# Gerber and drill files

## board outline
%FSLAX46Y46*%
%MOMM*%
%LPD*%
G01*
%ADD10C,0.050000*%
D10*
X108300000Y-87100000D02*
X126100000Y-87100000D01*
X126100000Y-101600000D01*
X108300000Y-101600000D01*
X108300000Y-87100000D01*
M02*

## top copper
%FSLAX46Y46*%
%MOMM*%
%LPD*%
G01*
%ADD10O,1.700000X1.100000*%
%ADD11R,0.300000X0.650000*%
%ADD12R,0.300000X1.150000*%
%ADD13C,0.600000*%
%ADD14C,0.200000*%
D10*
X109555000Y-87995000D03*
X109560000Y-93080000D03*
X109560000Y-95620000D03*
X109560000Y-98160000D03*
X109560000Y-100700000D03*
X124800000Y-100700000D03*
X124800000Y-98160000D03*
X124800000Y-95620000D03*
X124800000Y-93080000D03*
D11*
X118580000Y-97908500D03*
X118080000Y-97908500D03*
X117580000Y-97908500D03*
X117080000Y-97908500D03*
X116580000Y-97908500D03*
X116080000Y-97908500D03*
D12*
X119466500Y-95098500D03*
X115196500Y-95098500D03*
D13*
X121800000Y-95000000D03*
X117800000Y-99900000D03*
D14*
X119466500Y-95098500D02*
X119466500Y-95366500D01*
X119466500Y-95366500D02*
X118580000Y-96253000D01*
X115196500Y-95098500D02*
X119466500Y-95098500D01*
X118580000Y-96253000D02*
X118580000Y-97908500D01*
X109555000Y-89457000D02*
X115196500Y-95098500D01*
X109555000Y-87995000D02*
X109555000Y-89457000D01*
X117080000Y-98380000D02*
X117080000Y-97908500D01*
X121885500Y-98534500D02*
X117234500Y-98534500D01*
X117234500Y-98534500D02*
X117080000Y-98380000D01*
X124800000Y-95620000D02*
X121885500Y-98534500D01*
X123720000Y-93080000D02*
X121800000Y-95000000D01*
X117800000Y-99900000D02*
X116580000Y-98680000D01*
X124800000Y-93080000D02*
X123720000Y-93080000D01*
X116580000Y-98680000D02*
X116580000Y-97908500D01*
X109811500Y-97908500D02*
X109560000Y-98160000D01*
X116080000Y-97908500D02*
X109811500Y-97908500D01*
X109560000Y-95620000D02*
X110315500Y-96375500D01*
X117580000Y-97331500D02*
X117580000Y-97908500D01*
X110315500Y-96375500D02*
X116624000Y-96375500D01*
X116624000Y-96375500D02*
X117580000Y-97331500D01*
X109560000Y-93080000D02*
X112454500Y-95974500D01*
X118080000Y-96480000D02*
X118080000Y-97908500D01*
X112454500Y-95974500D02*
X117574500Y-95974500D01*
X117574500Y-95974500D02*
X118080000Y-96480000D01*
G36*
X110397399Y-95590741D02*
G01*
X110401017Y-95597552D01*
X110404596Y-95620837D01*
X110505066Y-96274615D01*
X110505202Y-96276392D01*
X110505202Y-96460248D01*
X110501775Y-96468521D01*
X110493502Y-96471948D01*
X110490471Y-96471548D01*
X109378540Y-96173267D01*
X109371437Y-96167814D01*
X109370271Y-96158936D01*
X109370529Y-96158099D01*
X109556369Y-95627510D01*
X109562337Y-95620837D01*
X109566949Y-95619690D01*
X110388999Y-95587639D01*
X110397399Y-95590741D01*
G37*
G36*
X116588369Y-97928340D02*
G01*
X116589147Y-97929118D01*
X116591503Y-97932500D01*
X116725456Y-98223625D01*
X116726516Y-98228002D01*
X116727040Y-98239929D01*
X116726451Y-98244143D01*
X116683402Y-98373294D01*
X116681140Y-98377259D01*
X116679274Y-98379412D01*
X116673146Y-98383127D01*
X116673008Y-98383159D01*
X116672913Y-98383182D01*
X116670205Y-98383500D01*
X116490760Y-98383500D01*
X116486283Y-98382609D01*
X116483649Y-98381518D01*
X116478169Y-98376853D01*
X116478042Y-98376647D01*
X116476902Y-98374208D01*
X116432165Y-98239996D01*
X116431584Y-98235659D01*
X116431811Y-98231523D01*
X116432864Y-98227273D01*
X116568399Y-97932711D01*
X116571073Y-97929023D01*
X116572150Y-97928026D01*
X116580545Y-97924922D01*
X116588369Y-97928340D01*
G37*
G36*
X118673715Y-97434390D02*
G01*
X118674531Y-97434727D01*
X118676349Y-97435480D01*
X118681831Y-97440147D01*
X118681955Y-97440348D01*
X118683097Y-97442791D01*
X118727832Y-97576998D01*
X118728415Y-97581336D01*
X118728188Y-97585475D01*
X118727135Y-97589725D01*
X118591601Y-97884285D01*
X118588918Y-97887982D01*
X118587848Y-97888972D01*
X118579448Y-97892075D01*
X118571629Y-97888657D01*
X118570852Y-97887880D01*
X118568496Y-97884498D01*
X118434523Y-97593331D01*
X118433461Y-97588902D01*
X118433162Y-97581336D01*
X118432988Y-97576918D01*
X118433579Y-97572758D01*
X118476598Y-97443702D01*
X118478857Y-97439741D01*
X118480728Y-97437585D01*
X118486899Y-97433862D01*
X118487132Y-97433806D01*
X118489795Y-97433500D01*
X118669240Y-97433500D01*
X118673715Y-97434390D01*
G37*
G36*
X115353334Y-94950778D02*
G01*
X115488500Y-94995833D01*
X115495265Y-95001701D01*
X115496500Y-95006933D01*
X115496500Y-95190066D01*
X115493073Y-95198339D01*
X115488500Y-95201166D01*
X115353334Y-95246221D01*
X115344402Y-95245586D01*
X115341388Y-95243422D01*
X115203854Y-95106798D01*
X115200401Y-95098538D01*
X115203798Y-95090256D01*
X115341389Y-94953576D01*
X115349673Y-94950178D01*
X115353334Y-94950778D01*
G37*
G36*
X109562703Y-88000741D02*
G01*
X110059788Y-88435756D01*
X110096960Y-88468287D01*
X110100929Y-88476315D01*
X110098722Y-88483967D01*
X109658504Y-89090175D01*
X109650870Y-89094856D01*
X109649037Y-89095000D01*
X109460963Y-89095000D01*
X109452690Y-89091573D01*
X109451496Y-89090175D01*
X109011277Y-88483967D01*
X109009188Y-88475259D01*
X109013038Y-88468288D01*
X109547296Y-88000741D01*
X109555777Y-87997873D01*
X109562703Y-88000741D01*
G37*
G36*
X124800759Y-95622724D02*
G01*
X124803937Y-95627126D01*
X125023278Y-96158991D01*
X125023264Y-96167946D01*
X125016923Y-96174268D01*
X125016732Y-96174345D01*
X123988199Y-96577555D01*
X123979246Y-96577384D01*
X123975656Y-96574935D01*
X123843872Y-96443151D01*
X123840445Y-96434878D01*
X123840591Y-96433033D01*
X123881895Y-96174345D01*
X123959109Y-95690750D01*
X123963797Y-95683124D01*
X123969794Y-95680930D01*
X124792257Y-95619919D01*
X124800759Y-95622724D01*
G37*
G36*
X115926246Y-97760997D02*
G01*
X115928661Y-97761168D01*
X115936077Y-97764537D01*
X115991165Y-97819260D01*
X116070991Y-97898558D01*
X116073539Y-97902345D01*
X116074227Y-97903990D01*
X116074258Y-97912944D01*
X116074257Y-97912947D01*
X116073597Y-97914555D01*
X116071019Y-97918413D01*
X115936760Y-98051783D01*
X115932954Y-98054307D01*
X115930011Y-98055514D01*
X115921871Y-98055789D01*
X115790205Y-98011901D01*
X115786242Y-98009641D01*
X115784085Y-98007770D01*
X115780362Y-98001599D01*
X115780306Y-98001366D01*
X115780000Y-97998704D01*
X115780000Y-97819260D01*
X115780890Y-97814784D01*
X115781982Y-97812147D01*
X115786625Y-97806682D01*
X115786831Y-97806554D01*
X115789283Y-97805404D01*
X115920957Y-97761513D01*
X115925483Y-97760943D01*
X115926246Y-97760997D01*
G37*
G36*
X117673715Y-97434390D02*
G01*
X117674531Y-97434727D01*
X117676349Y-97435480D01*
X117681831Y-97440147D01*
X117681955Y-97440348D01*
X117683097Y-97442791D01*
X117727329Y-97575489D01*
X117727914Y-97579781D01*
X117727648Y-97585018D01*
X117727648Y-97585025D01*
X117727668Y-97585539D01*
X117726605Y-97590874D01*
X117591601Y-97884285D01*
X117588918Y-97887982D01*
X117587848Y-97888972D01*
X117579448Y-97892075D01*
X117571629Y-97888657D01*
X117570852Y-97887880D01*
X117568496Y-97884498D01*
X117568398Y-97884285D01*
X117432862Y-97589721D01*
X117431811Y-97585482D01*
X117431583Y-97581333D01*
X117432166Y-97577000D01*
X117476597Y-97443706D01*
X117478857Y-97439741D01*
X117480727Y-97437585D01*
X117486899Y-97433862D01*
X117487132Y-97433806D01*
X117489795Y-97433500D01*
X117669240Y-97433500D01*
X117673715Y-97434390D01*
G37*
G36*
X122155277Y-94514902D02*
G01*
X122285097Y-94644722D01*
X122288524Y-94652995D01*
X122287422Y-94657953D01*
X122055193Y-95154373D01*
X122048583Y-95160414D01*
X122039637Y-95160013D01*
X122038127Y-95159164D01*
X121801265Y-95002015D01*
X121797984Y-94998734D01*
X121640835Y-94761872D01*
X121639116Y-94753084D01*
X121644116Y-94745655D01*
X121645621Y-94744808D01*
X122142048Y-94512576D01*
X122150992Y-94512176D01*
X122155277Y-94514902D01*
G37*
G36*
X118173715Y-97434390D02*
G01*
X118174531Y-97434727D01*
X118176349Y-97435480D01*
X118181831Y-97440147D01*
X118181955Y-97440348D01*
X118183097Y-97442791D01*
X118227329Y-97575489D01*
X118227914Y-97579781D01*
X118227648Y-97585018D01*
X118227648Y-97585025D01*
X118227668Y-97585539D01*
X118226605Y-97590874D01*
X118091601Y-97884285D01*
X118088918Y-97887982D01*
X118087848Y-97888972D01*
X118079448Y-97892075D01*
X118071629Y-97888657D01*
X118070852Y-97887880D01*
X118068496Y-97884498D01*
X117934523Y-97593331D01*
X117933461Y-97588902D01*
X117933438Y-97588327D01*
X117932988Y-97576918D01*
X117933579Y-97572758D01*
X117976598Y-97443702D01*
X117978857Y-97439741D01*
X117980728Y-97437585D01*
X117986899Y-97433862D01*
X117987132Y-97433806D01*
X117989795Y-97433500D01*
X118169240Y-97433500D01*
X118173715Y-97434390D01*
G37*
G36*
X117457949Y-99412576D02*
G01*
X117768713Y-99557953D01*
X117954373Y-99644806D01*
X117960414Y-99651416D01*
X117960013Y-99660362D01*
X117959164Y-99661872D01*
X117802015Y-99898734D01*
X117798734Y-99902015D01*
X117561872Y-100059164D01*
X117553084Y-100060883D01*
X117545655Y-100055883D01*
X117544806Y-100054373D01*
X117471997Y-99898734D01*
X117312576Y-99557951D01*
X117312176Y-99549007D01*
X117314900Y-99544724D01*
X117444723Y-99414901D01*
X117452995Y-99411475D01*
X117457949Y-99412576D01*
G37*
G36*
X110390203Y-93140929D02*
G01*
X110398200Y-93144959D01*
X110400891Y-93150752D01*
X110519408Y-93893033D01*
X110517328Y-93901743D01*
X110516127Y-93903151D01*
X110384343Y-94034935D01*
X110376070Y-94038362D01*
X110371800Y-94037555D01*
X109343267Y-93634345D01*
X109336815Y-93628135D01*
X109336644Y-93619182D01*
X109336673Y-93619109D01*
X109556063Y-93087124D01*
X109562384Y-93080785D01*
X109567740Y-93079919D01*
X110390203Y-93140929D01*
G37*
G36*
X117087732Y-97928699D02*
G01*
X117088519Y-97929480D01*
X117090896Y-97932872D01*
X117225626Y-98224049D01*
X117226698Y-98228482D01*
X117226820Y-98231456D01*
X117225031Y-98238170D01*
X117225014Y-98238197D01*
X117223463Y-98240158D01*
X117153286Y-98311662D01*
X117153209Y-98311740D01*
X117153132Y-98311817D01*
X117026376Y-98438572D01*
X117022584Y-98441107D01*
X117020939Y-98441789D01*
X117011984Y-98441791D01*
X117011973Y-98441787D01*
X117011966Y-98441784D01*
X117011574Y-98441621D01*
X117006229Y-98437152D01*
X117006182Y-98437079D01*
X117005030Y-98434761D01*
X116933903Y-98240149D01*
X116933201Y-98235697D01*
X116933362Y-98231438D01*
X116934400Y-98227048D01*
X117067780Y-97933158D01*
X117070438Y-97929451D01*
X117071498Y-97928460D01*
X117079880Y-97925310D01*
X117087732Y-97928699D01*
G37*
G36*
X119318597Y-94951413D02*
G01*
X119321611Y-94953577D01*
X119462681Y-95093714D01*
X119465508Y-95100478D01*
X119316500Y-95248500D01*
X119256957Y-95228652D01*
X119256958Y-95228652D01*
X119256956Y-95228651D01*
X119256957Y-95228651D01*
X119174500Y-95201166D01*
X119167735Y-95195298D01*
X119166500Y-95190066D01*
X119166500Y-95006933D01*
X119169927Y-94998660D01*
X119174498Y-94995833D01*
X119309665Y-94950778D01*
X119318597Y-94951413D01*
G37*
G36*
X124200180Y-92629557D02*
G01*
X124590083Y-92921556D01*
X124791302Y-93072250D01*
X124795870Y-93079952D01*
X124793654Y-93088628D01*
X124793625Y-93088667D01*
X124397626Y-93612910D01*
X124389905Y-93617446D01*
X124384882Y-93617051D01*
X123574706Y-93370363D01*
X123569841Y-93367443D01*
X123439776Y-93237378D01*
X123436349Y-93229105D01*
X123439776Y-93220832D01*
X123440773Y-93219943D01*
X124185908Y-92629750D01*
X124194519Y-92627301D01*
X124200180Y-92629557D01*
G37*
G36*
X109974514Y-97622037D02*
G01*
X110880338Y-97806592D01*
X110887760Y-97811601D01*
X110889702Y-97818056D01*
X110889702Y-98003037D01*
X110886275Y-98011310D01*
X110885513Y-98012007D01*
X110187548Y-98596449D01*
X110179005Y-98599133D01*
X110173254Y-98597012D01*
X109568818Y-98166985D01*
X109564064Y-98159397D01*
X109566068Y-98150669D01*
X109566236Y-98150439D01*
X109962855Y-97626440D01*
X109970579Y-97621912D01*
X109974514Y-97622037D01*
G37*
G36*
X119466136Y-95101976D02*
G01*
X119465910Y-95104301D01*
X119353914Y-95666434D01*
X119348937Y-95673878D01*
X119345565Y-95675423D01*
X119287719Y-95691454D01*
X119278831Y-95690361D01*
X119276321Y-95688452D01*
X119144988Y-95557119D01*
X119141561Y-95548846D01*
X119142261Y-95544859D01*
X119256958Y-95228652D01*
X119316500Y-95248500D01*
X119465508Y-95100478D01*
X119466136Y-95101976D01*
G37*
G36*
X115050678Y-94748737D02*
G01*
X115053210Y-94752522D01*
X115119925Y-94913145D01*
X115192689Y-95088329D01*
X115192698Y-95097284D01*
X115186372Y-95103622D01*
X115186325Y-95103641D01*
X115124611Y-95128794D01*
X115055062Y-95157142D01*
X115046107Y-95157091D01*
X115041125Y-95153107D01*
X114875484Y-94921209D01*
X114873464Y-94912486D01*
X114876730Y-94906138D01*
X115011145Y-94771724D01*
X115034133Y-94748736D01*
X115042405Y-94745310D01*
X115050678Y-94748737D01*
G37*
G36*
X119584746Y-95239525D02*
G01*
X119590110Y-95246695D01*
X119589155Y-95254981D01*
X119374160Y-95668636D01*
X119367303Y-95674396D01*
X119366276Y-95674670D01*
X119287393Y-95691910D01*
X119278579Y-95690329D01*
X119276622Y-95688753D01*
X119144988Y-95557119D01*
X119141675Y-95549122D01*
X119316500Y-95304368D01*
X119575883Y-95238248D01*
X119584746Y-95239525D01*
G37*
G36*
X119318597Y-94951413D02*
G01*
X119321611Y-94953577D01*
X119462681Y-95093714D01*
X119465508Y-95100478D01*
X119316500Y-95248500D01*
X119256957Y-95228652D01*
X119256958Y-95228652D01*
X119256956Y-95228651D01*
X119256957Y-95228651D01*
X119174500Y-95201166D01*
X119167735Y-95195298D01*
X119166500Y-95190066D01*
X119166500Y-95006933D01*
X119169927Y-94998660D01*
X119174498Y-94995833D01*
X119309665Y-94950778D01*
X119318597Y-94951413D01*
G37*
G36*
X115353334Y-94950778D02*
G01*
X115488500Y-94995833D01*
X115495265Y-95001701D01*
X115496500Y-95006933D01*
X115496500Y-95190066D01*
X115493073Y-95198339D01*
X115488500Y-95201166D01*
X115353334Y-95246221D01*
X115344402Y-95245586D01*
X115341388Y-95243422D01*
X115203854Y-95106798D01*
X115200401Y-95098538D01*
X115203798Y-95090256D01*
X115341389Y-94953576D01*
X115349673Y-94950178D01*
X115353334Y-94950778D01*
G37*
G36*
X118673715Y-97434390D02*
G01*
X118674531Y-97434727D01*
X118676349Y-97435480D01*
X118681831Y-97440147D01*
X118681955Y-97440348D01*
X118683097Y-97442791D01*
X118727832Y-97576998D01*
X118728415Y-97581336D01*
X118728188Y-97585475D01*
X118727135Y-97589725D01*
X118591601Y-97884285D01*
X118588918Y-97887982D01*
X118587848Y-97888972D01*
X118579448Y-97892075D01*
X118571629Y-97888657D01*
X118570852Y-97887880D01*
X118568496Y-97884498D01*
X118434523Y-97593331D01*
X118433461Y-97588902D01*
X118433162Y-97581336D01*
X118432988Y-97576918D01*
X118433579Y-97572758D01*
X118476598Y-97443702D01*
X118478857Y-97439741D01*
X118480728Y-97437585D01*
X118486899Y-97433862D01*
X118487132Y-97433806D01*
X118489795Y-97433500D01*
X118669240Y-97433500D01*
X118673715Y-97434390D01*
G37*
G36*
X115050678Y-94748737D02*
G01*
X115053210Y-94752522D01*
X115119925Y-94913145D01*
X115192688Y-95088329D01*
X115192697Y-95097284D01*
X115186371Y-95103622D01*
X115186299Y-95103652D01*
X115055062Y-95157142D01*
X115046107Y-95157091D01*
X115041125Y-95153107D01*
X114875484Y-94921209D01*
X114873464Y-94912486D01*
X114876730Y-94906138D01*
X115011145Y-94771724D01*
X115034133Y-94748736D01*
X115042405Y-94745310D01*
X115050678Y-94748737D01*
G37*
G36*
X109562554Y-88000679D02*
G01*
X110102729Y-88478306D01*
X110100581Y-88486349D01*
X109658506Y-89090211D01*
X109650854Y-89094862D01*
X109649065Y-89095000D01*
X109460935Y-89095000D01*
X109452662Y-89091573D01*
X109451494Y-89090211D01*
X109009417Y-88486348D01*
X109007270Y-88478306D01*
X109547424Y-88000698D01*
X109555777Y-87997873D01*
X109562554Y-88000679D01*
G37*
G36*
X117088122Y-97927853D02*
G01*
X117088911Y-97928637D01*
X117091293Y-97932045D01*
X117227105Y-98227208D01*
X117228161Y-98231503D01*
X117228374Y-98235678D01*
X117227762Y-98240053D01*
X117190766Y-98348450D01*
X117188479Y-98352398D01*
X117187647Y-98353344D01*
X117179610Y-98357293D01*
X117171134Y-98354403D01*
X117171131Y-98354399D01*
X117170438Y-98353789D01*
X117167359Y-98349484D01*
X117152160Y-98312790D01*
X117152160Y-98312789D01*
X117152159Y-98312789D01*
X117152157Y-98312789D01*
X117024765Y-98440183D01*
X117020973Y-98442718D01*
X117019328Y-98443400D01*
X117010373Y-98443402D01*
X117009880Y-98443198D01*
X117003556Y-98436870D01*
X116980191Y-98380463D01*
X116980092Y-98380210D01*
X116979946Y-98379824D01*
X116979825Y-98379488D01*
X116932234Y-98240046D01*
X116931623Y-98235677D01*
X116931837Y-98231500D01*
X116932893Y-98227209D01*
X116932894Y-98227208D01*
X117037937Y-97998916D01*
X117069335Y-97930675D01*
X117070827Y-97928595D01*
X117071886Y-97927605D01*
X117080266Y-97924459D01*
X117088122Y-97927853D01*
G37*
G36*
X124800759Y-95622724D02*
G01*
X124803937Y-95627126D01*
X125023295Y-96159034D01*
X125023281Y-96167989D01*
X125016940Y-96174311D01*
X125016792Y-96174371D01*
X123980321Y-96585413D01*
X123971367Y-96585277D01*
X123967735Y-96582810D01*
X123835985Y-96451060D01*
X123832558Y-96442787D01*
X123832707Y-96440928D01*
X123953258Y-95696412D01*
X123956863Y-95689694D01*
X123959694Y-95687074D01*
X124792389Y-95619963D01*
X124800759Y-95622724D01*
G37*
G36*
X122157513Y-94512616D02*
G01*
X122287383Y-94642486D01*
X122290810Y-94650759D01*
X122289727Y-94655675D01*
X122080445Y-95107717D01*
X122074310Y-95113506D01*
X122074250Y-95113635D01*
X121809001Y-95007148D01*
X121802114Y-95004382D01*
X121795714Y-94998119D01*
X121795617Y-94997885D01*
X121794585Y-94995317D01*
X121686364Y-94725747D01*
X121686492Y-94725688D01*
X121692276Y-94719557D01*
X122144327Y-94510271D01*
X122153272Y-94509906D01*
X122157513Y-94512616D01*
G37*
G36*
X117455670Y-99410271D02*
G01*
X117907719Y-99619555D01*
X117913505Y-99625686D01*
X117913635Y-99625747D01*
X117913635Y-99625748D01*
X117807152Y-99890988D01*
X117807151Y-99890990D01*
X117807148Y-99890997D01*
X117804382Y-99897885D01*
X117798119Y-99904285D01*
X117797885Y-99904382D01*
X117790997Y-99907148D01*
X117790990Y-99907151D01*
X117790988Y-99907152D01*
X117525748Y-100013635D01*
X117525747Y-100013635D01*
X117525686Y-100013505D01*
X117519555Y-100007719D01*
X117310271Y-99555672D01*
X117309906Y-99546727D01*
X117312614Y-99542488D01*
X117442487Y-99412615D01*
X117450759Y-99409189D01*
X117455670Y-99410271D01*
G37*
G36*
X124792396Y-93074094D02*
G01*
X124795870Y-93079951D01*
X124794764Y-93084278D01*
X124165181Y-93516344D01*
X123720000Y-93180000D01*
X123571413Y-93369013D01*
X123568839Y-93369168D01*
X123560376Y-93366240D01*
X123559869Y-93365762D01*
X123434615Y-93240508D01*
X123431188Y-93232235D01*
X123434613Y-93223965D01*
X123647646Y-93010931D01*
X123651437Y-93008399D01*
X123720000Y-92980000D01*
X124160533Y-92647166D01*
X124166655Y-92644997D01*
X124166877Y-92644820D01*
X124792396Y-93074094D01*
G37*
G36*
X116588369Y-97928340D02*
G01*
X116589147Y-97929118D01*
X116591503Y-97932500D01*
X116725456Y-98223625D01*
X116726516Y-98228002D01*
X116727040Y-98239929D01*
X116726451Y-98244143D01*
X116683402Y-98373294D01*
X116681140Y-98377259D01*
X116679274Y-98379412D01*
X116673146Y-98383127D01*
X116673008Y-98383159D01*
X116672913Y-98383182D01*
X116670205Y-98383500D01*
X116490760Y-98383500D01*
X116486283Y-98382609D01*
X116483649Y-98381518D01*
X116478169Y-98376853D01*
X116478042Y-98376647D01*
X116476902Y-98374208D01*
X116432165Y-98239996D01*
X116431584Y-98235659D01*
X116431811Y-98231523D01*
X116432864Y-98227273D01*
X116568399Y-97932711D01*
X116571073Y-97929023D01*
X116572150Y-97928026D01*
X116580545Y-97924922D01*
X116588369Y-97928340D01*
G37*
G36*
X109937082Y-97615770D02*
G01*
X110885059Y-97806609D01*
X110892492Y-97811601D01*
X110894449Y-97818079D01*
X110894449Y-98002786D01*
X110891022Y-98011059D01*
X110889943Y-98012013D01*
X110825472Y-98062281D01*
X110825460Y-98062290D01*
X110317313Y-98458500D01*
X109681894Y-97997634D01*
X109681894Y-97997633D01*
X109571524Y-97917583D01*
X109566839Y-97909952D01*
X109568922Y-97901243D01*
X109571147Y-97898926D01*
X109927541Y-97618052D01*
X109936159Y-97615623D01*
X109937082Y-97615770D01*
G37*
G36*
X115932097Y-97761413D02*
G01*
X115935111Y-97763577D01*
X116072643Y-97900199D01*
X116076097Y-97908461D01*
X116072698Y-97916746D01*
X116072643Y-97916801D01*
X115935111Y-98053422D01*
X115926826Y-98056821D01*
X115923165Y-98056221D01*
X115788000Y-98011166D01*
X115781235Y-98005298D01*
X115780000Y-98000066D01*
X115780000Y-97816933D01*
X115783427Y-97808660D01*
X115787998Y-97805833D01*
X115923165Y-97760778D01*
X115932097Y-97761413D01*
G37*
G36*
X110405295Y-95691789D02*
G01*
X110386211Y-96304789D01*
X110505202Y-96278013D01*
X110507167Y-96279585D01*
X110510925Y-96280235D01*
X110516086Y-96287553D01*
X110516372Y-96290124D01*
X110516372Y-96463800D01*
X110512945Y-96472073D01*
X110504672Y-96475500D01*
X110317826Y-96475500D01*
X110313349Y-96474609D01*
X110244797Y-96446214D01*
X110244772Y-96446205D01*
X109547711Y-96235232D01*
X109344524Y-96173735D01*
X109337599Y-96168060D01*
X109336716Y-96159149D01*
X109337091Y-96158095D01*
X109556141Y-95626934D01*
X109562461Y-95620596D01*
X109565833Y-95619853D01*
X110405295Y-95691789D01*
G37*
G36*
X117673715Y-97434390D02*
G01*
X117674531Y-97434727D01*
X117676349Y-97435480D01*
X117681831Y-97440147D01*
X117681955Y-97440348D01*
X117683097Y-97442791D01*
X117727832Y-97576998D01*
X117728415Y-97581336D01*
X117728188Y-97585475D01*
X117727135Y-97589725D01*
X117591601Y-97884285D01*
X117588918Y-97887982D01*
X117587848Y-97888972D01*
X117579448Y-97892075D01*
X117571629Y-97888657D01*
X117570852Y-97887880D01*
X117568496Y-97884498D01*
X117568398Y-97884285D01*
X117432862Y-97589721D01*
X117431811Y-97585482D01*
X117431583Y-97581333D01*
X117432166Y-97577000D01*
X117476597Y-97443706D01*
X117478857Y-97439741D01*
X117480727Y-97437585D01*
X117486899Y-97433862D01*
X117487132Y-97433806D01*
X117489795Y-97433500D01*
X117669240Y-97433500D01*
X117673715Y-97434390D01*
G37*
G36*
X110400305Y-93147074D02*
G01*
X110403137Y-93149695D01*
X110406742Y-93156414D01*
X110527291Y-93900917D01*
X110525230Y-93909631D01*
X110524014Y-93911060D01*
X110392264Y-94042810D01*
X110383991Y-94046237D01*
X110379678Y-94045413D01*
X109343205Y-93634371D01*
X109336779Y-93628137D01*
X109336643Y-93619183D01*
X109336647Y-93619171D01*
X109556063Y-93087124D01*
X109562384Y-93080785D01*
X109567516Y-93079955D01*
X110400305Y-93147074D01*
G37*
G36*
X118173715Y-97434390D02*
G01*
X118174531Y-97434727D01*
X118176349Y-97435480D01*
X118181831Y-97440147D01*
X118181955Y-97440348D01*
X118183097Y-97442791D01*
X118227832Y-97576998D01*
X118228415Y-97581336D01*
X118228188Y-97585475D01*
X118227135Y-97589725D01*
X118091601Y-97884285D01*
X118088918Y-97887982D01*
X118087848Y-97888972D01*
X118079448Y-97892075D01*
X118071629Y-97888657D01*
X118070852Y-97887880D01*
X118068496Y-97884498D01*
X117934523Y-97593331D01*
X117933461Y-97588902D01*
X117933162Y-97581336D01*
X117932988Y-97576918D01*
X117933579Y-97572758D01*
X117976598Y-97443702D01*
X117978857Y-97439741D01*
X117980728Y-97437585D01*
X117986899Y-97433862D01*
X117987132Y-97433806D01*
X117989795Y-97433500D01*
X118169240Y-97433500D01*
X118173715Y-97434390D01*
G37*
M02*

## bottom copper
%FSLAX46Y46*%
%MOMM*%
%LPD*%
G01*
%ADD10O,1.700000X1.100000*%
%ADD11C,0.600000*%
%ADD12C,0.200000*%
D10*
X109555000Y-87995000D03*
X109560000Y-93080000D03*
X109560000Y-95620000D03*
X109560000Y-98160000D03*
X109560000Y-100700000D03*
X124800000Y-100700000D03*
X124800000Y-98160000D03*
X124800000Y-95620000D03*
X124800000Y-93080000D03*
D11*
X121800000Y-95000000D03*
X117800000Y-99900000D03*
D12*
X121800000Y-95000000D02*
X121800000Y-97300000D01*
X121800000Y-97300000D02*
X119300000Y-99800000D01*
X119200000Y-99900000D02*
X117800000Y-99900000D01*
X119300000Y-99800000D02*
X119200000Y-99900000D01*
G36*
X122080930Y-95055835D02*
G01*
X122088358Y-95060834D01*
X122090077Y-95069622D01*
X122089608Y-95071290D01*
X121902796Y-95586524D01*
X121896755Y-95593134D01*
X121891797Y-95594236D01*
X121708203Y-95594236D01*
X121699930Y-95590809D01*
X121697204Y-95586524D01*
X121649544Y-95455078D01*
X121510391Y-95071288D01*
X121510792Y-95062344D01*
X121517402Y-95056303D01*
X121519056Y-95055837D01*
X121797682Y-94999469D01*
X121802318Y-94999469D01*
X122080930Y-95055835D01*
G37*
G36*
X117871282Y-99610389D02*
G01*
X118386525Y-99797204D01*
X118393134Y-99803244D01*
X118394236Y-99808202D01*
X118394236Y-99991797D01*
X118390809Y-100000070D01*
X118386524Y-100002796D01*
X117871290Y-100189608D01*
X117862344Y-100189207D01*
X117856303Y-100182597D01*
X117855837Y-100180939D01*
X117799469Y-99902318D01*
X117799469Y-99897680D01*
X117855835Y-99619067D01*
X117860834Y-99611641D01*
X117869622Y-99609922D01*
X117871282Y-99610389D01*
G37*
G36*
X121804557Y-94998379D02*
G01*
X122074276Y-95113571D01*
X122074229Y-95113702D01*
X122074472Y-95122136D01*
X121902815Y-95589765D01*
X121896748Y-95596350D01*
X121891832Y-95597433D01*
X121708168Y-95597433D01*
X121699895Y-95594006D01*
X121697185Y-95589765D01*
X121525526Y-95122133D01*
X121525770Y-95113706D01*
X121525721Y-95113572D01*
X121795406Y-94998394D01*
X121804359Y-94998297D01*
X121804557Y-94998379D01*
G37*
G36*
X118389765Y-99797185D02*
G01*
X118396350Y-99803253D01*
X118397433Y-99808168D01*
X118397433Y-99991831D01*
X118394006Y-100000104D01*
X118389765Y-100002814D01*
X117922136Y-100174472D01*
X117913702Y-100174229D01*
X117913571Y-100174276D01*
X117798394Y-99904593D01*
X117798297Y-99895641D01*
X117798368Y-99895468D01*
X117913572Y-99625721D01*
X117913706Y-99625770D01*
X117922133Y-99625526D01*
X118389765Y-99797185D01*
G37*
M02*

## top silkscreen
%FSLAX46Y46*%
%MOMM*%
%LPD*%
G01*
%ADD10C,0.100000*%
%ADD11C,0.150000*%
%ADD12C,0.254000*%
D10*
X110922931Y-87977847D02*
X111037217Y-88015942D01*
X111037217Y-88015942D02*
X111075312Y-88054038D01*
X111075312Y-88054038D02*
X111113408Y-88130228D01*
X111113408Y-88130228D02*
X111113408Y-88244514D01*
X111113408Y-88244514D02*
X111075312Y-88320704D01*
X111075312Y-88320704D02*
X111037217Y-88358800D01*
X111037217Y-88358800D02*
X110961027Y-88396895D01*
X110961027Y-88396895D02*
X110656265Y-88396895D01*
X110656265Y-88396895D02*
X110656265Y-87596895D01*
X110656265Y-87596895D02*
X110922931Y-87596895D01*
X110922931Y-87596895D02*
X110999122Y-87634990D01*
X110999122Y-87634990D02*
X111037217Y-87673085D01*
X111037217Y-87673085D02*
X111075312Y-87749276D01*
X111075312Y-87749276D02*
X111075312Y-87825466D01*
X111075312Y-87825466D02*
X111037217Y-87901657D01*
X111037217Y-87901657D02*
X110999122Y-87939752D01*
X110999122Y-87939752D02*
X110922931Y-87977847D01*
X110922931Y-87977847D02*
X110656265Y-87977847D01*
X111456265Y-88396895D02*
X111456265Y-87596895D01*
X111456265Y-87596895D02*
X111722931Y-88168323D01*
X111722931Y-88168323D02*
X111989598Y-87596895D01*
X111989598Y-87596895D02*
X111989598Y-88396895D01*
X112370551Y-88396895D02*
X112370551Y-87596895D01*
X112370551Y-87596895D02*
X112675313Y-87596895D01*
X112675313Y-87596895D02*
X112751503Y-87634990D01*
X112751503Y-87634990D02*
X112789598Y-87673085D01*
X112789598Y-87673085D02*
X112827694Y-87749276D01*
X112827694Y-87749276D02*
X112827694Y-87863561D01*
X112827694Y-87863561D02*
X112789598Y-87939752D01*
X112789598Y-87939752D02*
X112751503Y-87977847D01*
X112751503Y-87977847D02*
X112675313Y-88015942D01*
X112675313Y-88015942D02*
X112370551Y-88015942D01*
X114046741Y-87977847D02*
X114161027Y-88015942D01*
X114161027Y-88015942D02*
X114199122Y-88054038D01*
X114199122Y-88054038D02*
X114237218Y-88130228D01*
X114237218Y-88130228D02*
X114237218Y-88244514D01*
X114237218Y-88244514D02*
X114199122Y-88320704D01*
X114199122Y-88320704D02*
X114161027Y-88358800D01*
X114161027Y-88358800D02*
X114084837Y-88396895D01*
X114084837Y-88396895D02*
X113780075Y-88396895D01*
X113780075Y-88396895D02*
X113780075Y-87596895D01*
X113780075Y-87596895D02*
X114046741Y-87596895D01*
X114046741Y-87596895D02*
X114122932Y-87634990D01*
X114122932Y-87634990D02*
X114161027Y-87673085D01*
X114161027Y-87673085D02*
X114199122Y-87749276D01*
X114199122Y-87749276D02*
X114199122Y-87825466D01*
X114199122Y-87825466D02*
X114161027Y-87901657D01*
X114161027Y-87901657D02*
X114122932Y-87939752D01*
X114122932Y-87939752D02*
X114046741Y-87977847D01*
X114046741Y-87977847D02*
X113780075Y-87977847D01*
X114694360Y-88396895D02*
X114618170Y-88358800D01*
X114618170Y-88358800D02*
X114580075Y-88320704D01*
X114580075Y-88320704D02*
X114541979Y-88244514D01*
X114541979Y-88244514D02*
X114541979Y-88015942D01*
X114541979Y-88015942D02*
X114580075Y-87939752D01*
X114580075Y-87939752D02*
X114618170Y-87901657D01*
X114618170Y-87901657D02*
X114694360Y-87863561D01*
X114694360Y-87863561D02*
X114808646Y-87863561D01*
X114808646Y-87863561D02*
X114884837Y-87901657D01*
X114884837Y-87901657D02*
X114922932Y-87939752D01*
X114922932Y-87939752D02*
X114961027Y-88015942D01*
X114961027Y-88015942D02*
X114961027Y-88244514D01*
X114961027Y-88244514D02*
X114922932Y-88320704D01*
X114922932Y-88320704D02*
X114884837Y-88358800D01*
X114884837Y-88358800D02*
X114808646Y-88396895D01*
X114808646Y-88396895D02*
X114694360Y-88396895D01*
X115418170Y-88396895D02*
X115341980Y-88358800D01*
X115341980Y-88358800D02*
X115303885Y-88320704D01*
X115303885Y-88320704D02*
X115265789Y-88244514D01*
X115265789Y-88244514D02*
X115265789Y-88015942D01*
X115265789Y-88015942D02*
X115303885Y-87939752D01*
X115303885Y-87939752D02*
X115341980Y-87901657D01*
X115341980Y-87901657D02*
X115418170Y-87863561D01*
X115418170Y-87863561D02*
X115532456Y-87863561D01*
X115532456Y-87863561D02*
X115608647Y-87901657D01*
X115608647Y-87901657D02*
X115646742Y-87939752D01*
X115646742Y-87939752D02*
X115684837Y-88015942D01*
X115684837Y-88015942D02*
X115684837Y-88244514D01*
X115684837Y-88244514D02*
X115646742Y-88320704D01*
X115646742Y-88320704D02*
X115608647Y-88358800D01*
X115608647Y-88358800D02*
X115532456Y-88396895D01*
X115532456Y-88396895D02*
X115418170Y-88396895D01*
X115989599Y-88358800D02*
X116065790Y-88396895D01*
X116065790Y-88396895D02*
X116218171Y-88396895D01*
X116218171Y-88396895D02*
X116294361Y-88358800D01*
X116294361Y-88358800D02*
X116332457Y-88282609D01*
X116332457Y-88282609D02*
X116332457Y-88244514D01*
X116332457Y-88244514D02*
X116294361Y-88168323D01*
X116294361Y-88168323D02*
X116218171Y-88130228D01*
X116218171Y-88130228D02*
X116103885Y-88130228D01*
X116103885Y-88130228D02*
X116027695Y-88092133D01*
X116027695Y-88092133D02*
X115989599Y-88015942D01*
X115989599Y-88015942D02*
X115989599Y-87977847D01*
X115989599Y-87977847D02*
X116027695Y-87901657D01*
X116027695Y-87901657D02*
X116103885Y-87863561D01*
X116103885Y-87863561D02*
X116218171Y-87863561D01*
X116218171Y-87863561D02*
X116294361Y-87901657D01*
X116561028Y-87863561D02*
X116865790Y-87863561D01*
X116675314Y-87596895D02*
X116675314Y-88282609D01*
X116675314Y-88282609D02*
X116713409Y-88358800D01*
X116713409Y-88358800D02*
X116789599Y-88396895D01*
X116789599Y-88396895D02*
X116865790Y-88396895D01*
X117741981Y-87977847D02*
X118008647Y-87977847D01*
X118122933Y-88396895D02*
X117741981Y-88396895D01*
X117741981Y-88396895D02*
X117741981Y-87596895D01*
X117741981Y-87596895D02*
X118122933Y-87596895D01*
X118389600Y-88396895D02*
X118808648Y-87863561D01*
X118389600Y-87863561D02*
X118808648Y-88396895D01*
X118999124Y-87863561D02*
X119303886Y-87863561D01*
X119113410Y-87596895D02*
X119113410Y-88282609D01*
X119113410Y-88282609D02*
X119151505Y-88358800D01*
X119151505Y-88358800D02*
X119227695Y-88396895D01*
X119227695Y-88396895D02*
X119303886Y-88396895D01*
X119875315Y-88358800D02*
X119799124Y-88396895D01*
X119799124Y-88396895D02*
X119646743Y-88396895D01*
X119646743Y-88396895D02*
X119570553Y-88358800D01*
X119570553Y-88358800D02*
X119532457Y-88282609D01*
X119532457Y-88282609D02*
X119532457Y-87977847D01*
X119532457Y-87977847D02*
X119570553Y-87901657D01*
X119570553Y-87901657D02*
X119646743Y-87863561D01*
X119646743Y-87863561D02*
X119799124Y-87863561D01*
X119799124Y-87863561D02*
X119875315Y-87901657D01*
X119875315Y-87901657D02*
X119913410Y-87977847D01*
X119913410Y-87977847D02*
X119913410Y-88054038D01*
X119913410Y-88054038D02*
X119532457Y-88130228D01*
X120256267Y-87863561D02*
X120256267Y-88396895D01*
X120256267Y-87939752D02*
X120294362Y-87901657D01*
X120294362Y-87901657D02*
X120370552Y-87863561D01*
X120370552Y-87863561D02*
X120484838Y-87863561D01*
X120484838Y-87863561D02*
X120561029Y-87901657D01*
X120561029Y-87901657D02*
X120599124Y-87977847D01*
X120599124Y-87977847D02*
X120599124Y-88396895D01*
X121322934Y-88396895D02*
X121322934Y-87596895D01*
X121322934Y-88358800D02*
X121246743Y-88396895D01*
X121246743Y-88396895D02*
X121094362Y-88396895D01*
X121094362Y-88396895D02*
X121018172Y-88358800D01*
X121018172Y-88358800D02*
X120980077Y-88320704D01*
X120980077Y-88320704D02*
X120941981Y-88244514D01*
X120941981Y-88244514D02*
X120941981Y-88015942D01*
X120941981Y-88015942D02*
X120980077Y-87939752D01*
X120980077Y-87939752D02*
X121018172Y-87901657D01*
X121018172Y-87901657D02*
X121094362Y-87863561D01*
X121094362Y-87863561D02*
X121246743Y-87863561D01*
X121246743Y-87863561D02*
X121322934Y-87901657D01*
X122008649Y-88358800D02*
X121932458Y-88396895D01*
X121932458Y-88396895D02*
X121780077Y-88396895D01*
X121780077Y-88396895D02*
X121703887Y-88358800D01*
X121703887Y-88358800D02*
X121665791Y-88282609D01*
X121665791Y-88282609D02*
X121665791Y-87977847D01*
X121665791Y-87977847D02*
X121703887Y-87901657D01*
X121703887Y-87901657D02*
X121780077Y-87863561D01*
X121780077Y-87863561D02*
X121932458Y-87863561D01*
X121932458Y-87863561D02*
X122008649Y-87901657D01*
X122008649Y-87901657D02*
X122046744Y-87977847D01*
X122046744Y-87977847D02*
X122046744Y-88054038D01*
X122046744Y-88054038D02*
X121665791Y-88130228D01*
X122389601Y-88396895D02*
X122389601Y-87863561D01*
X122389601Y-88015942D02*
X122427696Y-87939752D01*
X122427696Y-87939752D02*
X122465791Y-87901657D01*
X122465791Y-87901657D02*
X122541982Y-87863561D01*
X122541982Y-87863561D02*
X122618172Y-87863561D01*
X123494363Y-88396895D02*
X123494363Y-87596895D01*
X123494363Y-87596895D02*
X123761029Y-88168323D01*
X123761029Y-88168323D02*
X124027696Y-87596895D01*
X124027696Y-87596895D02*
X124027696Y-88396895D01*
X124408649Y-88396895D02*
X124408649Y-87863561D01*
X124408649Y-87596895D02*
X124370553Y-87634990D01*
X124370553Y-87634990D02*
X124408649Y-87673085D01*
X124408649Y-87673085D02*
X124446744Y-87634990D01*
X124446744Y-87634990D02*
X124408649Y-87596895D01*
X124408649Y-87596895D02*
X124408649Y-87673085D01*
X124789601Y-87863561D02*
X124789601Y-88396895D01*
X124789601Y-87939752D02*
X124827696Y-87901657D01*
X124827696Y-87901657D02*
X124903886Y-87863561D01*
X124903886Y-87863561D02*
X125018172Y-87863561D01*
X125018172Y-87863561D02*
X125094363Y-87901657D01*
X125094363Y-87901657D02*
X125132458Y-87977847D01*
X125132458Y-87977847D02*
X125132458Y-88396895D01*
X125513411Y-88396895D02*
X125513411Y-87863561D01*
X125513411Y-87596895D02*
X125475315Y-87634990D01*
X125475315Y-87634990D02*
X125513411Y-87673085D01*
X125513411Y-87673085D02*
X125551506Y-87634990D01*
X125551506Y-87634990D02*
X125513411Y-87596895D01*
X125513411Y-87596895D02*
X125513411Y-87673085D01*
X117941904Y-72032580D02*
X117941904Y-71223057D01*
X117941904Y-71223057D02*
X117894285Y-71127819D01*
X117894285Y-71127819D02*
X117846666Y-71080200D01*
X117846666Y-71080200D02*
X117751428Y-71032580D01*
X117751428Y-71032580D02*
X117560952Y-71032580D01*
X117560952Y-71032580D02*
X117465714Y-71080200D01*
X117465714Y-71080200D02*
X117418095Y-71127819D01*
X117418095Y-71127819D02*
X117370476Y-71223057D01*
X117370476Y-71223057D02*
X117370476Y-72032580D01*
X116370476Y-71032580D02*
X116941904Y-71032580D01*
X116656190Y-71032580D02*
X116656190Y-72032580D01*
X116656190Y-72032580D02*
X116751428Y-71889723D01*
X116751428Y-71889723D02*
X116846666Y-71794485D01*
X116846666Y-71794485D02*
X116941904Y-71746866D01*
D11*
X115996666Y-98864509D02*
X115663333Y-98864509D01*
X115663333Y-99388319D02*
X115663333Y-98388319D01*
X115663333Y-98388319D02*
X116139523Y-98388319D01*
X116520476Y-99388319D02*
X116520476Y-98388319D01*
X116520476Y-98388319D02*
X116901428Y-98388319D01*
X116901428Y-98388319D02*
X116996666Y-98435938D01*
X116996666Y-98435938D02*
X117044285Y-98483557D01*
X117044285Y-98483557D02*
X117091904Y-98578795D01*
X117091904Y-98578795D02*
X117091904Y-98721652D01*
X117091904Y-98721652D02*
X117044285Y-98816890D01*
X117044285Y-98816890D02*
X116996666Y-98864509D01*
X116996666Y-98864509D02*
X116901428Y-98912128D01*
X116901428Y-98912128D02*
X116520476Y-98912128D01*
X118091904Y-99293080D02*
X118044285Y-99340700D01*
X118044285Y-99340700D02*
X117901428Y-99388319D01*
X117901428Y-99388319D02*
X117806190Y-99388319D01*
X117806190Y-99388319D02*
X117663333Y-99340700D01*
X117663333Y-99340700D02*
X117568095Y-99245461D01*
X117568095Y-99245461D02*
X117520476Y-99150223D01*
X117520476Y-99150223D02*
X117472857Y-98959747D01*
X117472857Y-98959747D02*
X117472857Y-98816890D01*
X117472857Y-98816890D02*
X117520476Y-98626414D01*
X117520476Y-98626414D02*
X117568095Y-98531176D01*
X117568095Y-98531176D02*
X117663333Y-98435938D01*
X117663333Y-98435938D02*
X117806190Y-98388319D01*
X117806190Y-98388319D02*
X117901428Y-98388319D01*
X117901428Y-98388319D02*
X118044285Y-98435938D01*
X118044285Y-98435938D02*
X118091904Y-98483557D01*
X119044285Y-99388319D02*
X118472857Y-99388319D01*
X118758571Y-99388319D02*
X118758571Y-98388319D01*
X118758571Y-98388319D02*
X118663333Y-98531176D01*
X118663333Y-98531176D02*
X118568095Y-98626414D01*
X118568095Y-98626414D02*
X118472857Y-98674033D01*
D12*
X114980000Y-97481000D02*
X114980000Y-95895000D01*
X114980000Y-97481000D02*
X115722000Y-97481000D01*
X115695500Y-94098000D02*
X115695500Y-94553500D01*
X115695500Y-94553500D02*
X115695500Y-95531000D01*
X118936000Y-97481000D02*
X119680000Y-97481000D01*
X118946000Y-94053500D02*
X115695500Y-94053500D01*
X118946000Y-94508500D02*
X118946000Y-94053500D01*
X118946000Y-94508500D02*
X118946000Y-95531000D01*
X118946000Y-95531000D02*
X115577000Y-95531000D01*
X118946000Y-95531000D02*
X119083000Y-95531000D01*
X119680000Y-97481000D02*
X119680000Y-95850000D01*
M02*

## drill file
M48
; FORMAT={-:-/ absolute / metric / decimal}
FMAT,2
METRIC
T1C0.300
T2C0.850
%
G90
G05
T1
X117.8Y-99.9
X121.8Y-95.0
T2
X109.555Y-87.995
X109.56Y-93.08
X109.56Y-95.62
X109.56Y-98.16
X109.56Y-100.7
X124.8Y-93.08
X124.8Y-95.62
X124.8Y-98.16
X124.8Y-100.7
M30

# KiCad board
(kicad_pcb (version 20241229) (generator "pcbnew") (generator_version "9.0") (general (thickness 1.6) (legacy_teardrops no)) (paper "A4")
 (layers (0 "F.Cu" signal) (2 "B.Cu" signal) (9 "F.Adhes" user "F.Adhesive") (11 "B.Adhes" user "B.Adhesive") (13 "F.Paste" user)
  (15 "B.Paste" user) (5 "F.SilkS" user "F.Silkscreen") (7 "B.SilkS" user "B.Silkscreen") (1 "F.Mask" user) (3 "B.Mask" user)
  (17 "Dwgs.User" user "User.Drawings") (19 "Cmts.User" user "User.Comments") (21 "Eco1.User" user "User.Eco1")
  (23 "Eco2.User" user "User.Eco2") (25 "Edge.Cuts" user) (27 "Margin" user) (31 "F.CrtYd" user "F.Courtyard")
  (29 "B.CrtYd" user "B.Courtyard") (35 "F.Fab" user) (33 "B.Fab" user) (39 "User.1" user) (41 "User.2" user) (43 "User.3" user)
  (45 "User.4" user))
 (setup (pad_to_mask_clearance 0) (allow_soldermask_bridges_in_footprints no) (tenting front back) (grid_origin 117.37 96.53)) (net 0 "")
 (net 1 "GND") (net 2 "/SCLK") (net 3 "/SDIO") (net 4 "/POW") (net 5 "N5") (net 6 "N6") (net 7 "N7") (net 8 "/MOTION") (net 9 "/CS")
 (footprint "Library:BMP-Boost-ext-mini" (layer "F.Cu") (at 117.18 76.57)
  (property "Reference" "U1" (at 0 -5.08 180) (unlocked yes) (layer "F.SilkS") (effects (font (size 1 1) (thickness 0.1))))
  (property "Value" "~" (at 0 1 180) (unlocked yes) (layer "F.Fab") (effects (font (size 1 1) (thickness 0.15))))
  (pad "26" thru_hole oval (at -7.625 11.425 180) (size 1.7 1.1) (drill 0.85) (layers "*.Cu" "*.Mask") (remove_unused_layers no)
   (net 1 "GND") (thermal_bridge_angle 0)
   (teardrops (best_length_ratio 0.5) (max_length 1) (best_width_ratio 1) (max_width 2) (curved_edges no) (filter_ratio 0.9) (enabled yes)
    (allow_two_segments yes) (prefer_zone_connections yes)))
  (pad "31" thru_hole oval (at -7.62 16.51 180) (size 1.7 1.1) (drill 0.85) (layers "*.Cu" "*.Mask") (remove_unused_layers no)
   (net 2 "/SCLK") (thermal_bridge_angle 45)
   (teardrops (best_length_ratio 0.5) (max_length 1) (best_width_ratio 1) (max_width 2) (curved_edges no) (filter_ratio 0.9) (enabled yes)
    (allow_two_segments yes) (prefer_zone_connections yes)))
  (pad "32" thru_hole oval (at -7.62 19.05 180) (size 1.7 1.1) (drill 0.85) (layers "*.Cu" "*.Mask") (remove_unused_layers no)
   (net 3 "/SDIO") (thermal_bridge_angle 45)
   (teardrops (best_length_ratio 0.5) (max_length 1) (best_width_ratio 1) (max_width 2) (curved_edges no) (filter_ratio 0.9) (enabled yes)
    (allow_two_segments yes) (prefer_zone_connections yes)))
  (pad "33" thru_hole oval (at -7.62 21.59 180) (size 1.7 1.1) (drill 0.85) (layers "*.Cu" "*.Mask") (remove_unused_layers no)
   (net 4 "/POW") (thermal_bridge_angle 45)
   (teardrops (best_length_ratio 0.5) (max_length 1) (best_width_ratio 1) (max_width 2) (curved_edges no) (filter_ratio 0.9) (enabled yes)
    (allow_two_segments yes) (prefer_zone_connections yes)))
  (pad "34" thru_hole oval (at -7.62 24.13 180) (size 1.7 1.1) (drill 0.85) (layers "*.Cu" "*.Mask") (remove_unused_layers no) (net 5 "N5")
   (thermal_bridge_angle 45)
   (teardrops (best_length_ratio 0.5) (max_length 1) (best_width_ratio 1) (max_width 2) (curved_edges no) (filter_ratio 0.9) (enabled yes)
    (allow_two_segments yes) (prefer_zone_connections yes)))
  (pad "35" thru_hole oval (at 7.62 24.13 180) (size 1.7 1.1) (drill 0.85) (layers "*.Cu" "*.Mask") (remove_unused_layers no) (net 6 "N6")
   (thermal_bridge_angle 45)
   (teardrops (best_length_ratio 0.5) (max_length 1) (best_width_ratio 1) (max_width 2) (curved_edges no) (filter_ratio 0.9) (enabled yes)
    (allow_two_segments yes) (prefer_zone_connections yes)))
  (pad "36" thru_hole oval (at 7.62 21.59 180) (size 1.7 1.1) (drill 0.85) (layers "*.Cu" "*.Mask") (remove_unused_layers no) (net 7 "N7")
   (thermal_bridge_angle 45)
   (teardrops (best_length_ratio 0.5) (max_length 1) (best_width_ratio 1) (max_width 2) (curved_edges no) (filter_ratio 0.9) (enabled yes)
    (allow_two_segments yes) (prefer_zone_connections yes)))
  (pad "37" thru_hole oval (at 7.62 19.05 180) (size 1.7 1.1) (drill 0.85) (layers "*.Cu" "*.Mask") (remove_unused_layers no)
   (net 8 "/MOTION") (thermal_bridge_angle 45)
   (teardrops (best_length_ratio 0.5) (max_length 1) (best_width_ratio 1) (max_width 2) (curved_edges no) (filter_ratio 0.9) (enabled yes)
    (allow_two_segments yes) (prefer_zone_connections yes)))
  (pad "38" thru_hole oval (at 7.62 16.51 180) (size 1.7 1.1) (drill 0.85) (layers "*.Cu" "*.Mask") (remove_unused_layers no) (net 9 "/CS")
   (thermal_bridge_angle 45)
   (teardrops (best_length_ratio 0.5) (max_length 1) (best_width_ratio 1) (max_width 2) (curved_edges no) (filter_ratio 0.9) (enabled yes)
    (allow_two_segments yes) (prefer_zone_connections yes))))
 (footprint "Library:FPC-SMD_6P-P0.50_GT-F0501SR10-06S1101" (layer "F.Cu") (at 117.3315 96.5035 180)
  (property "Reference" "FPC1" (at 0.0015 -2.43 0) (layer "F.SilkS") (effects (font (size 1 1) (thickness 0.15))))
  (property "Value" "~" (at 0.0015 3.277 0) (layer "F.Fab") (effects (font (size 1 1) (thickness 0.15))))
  (fp_line (start 2.3515 -0.9775) (end 2.3515 0.6085) (stroke (width 0.254) (type default)) (layer "F.SilkS"))
  (fp_line (start 2.3515 -0.9775) (end 1.6095 -0.9775) (stroke (width 0.254) (type default)) (layer "F.SilkS"))
  (fp_line (start 1.636 2.4055) (end 1.636 1.95) (stroke (width 0.254) (type default)) (layer "F.SilkS"))
  (fp_line (start 1.636 1.95) (end 1.636 0.9725) (stroke (width 0.254) (type default)) (layer "F.SilkS"))
  (fp_line (start -1.6045 -0.9775) (end -2.3485 -0.9775) (stroke (width 0.254) (type default)) (layer "F.SilkS"))
  (fp_line (start -1.6145 2.45) (end 1.636 2.45) (stroke (width 0.254) (type default)) (layer "F.SilkS"))
  (fp_line (start -1.6145 1.995) (end -1.6145 2.45) (stroke (width 0.254) (type default)) (layer "F.SilkS"))
  (fp_line (start -1.6145 1.995) (end -1.6145 0.9725) (stroke (width 0.254) (type default)) (layer "F.SilkS"))
  (fp_line (start -1.6145 0.9725) (end 1.7545 0.9725) (stroke (width 0.254) (type default)) (layer "F.SilkS"))
  (fp_line (start -1.6145 0.9725) (end -1.7515 0.9725) (stroke (width 0.254) (type default)) (layer "F.SilkS"))
  (fp_line (start -2.3485 -0.9775) (end -2.3485 0.6535) (stroke (width 0.254) (type default)) (layer "F.SilkS"))
  (pad "1" smd rect (at -1.2485 -1.405 180) (size 0.3 0.65) (layers "F.Cu" "F.Mask" "F.Paste") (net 1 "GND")
   (teardrops (best_length_ratio 0.5) (max_length 1) (best_width_ratio 1) (max_width 2) (curved_edges no) (filter_ratio 0.9) (enabled yes)
    (allow_two_segments yes) (prefer_zone_connections yes)))
  (pad "2" smd rect (at -0.7485 -1.405 180) (size 0.3 0.65) (layers "F.Cu" "F.Mask" "F.Paste") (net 2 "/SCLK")
   (teardrops (best_length_ratio 0.5) (max_length 1) (best_width_ratio 1) (max_width 2) (curved_edges no) (filter_ratio 0.9) (enabled yes)
    (allow_two_segments yes) (prefer_zone_connections yes)))
  (pad "3" smd rect (at -0.2485 -1.405 180) (size 0.3 0.65) (layers "F.Cu" "F.Mask" "F.Paste") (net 3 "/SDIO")
   (teardrops (best_length_ratio 0.5) (max_length 1) (best_width_ratio 1) (max_width 2) (curved_edges no) (filter_ratio 0.9) (enabled yes)
    (allow_two_segments yes) (prefer_zone_connections yes)))
  (pad "4" smd rect (at 0.2515 -1.405 180) (size 0.3 0.65) (layers "F.Cu" "F.Mask" "F.Paste") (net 8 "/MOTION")
   (teardrops (best_length_ratio 0.5) (max_length 1) (best_width_ratio 1) (max_width 2) (curved_edges no) (filter_ratio 0.9) (enabled yes)
    (allow_two_segments yes) (prefer_zone_connections yes)))
  (pad "5" smd rect (at 0.7515 -1.405 180) (size 0.3 0.65) (layers "F.Cu" "F.Mask" "F.Paste") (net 9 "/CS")
   (teardrops (best_length_ratio 0.5) (max_length 1) (best_width_ratio 1) (max_width 2) (curved_edges no) (filter_ratio 0.9) (enabled yes)
    (allow_two_segments yes) (prefer_zone_connections yes)))
  (pad "6" smd rect (at 1.2515 -1.405 180) (size 0.3 0.65) (layers "F.Cu" "F.Mask" "F.Paste") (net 4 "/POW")
   (teardrops (best_length_ratio 0.5) (max_length 1) (best_width_ratio 1) (max_width 2) (curved_edges no) (filter_ratio 0.9) (enabled yes)
    (allow_two_segments yes) (prefer_zone_connections yes)))
  (pad "7" smd rect (at -2.135 1.405 180) (size 0.3 1.15) (layers "F.Cu" "F.Mask" "F.Paste") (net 1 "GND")
   (teardrops (best_length_ratio 0.5) (max_length 1) (best_width_ratio 1) (max_width 2) (curved_edges no) (filter_ratio 0.9) (enabled yes)
    (allow_two_segments yes) (prefer_zone_connections yes)))
  (pad "8" smd rect (at 2.135 1.405) (size 0.3 1.15) (layers "F.Cu" "F.Mask" "F.Paste") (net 1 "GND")
   (teardrops (best_length_ratio 0.5) (max_length 1) (best_width_ratio 1) (max_width 2) (curved_edges no) (filter_ratio 0.9) (enabled yes)
    (allow_two_segments yes) (prefer_zone_connections yes))))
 (gr_rect (start 108.3 87.1) (end 126.1 101.6) (stroke (width 0.05) (type solid)) (fill no) (layer "Edge.Cuts"))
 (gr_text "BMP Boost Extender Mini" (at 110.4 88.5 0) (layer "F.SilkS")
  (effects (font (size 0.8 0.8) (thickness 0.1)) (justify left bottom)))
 (segment (start 119.4665 95.0985) (end 119.4665 95.3665) (width 0.2) (layer "F.Cu") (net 1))
 (segment (start 119.4665 95.3665) (end 118.58 96.253) (width 0.2) (layer "F.Cu") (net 1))
 (segment (start 115.1965 95.0985) (end 119.4665 95.0985) (width 0.2) (layer "F.Cu") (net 1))
 (segment (start 118.58 96.253) (end 118.58 97.9085) (width 0.2) (layer "F.Cu") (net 1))
 (segment (start 109.555 89.457) (end 115.1965 95.0985) (width 0.2) (layer "F.Cu") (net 1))
 (segment (start 109.555 87.995) (end 109.555 89.457) (width 0.2) (layer "F.Cu") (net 1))
 (segment (start 117.08 98.38) (end 117.08 97.9085) (width 0.2) (layer "F.Cu") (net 8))
 (segment (start 121.8855 98.5345) (end 117.2345 98.5345) (width 0.2) (layer "F.Cu") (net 8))
 (segment (start 117.2345 98.5345) (end 117.08 98.38) (width 0.2) (layer "F.Cu") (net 8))
 (segment (start 124.8 95.62) (end 121.8855 98.5345) (width 0.2) (layer "F.Cu") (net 8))
 (segment (start 123.72 93.08) (end 121.8 95) (width 0.2) (layer "F.Cu") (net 9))
 (segment (start 117.8 99.9) (end 116.58 98.68) (width 0.2) (layer "F.Cu") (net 9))
 (segment (start 124.8 93.08) (end 123.72 93.08) (width 0.2) (layer "F.Cu") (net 9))
 (segment (start 116.58 98.68) (end 116.58 97.9085) (width 0.2) (layer "F.Cu") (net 9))
 (via (at 121.8 95) (size 0.6) (drill 0.3) (layers "F.Cu" "B.Cu")
  (teardrops (best_length_ratio 0.5) (max_length 1) (best_width_ratio 1) (max_width 2) (curved_edges no) (filter_ratio 0.9) (enabled yes)
   (allow_two_segments yes) (prefer_zone_connections yes))
  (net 9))
 (via (at 117.8 99.9) (size 0.6) (drill 0.3) (layers "F.Cu" "B.Cu")
  (teardrops (best_length_ratio 0.5) (max_length 1) (best_width_ratio 1) (max_width 2) (curved_edges no) (filter_ratio 0.9) (enabled yes)
   (allow_two_segments yes) (prefer_zone_connections yes))
  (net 9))
 (segment (start 121.8 95) (end 121.8 97.3) (width 0.2) (layer "B.Cu") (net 9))
 (segment (start 121.8 97.3) (end 119.3 99.8) (width 0.2) (layer "B.Cu") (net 9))
 (segment (start 119.2 99.9) (end 117.8 99.9) (width 0.2) (layer "B.Cu") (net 9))
 (segment (start 119.3 99.8) (end 119.2 99.9) (width 0.2) (layer "B.Cu") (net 9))
 (segment (start 109.8115 97.9085) (end 109.56 98.16) (width 0.2) (layer "F.Cu") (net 4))
 (segment (start 116.08 97.9085) (end 109.8115 97.9085) (width 0.2) (layer "F.Cu") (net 4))
 (segment (start 109.56 95.62) (end 110.3155 96.3755) (width 0.2) (layer "F.Cu") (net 3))
 (segment (start 117.58 97.3315) (end 117.58 97.9085) (width 0.2) (layer "F.Cu") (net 3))
 (segment (start 110.3155 96.3755) (end 116.624 96.3755) (width 0.2) (layer "F.Cu") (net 3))
 (segment (start 116.624 96.3755) (end 117.58 97.3315) (width 0.2) (layer "F.Cu") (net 3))
 (segment (start 109.56 93.08) (end 112.4545 95.9745) (width 0.2) (layer "F.Cu") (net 2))
 (segment (start 118.08 96.48) (end 118.08 97.9085) (width 0.2) (layer "F.Cu") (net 2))
 (segment (start 112.4545 95.9745) (end 117.5745 95.9745) (width 0.2) (layer "F.Cu") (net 2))
 (segment (start 117.5745 95.9745) (end 118.08 96.48) (width 0.2) (layer "F.Cu") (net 2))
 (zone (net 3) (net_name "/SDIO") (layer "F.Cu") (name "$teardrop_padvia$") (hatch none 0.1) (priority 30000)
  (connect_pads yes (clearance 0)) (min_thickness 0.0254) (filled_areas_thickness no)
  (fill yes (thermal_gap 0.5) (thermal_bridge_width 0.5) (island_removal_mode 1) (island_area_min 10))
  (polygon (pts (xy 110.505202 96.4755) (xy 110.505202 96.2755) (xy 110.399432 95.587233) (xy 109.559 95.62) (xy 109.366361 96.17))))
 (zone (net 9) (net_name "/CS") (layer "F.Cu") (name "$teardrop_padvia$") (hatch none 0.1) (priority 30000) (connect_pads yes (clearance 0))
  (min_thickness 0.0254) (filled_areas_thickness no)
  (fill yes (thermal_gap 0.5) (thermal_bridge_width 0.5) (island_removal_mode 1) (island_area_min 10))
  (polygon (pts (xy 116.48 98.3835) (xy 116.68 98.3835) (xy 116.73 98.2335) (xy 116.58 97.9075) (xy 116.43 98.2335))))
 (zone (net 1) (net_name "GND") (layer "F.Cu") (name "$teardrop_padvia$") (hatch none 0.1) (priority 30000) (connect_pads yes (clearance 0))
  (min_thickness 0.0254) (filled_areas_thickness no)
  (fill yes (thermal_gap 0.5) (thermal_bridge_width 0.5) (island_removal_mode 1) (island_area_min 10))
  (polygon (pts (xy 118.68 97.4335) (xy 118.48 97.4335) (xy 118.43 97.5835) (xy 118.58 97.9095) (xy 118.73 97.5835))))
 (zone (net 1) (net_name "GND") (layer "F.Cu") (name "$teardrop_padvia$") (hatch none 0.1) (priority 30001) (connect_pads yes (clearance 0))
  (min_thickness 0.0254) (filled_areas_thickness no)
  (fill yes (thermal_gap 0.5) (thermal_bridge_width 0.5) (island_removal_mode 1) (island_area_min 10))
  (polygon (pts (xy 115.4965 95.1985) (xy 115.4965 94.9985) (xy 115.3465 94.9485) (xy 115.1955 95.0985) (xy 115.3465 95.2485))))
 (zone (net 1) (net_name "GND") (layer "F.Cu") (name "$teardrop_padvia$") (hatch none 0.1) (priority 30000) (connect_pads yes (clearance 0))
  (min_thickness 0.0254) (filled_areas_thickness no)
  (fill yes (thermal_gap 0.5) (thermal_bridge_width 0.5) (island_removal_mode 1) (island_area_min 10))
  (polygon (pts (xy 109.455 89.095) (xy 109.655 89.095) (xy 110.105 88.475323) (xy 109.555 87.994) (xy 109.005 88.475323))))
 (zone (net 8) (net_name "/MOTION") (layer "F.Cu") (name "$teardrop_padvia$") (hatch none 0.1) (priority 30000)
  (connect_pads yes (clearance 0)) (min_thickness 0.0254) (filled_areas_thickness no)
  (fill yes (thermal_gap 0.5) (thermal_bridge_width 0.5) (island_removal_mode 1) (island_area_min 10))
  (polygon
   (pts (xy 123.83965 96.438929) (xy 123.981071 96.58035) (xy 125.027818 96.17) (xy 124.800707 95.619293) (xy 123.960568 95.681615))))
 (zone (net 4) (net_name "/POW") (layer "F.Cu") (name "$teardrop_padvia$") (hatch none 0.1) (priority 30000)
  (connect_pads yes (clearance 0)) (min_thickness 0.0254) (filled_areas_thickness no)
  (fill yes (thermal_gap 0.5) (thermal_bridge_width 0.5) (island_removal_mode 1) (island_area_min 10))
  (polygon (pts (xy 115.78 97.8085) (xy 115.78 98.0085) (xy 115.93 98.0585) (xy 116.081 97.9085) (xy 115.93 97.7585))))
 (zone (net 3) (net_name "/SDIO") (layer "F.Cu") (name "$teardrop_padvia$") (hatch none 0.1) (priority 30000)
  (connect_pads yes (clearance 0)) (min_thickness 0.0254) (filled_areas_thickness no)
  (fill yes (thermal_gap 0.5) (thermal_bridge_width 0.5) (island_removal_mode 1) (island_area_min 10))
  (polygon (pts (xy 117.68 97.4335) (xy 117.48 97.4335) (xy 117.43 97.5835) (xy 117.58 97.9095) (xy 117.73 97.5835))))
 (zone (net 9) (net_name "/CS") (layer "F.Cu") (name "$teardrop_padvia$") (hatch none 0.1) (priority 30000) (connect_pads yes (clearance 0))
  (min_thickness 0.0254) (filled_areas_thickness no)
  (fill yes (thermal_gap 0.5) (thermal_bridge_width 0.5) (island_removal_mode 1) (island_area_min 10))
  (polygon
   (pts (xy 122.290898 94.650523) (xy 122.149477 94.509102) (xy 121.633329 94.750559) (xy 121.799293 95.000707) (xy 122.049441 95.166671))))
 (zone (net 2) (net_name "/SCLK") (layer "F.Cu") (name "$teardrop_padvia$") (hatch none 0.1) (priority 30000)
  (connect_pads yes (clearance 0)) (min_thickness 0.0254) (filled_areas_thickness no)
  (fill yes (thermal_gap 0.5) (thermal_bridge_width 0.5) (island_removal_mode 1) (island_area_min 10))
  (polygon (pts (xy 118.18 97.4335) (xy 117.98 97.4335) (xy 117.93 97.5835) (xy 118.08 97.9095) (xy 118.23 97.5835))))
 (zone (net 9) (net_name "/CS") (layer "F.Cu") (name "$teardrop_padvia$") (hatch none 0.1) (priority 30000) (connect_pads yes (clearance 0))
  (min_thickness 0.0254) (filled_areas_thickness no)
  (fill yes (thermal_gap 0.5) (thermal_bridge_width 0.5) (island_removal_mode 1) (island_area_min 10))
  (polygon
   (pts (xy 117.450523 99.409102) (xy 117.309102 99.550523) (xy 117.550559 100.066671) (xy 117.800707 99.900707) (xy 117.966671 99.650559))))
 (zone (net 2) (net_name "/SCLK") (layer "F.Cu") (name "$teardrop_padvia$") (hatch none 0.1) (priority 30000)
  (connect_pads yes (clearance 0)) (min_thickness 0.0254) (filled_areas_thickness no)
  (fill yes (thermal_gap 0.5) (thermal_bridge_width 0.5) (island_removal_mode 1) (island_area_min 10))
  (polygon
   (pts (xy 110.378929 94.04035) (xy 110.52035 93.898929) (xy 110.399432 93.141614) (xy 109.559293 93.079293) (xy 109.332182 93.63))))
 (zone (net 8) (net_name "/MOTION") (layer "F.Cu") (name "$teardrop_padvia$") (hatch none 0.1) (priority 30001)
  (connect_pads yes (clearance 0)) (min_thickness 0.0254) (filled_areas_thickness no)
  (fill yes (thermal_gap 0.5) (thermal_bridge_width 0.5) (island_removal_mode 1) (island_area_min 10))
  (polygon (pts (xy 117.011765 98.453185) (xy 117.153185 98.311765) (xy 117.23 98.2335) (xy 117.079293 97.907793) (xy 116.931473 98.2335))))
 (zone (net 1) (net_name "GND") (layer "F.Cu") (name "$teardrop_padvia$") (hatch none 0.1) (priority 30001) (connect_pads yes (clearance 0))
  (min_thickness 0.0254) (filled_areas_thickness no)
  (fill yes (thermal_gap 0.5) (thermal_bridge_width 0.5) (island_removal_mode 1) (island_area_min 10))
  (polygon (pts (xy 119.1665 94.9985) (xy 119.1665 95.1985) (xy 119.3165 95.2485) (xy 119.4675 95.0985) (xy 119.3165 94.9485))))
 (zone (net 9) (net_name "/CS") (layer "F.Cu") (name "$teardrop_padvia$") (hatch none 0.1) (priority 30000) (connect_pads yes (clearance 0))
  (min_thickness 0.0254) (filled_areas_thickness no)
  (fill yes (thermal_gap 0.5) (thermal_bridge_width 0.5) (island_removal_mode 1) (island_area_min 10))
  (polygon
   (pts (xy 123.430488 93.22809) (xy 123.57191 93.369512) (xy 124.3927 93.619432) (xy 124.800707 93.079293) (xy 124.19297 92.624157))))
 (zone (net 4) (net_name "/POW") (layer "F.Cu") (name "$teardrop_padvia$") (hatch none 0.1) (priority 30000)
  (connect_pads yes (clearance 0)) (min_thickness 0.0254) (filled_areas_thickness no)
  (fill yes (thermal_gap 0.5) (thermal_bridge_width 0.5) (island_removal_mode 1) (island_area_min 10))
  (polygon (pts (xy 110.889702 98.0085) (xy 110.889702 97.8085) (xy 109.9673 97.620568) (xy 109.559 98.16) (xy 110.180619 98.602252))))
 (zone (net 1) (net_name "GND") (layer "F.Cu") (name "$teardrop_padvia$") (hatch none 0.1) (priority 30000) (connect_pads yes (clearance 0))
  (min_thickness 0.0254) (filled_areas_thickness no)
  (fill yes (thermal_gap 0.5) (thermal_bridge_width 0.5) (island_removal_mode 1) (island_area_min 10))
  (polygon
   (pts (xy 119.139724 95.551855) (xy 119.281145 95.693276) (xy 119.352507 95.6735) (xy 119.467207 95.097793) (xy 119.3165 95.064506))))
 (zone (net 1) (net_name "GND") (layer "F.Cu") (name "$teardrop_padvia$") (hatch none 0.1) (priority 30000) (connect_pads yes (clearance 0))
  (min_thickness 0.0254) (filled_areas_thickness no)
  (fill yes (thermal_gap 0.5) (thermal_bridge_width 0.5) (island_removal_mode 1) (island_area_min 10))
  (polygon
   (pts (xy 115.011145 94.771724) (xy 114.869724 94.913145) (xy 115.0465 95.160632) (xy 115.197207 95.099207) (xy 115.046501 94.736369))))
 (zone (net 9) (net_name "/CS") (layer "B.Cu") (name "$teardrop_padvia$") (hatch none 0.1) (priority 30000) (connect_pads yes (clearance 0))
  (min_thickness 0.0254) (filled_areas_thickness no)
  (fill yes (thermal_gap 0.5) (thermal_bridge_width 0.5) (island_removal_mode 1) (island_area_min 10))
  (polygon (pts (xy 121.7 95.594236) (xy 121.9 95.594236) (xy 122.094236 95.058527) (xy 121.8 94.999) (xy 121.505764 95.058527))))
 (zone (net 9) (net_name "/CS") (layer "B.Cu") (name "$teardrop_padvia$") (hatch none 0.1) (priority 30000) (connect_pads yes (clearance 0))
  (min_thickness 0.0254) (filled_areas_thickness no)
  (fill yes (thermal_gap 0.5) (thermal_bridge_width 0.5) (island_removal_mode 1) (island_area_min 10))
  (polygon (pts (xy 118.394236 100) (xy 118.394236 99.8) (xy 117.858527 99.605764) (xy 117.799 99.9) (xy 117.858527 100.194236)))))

